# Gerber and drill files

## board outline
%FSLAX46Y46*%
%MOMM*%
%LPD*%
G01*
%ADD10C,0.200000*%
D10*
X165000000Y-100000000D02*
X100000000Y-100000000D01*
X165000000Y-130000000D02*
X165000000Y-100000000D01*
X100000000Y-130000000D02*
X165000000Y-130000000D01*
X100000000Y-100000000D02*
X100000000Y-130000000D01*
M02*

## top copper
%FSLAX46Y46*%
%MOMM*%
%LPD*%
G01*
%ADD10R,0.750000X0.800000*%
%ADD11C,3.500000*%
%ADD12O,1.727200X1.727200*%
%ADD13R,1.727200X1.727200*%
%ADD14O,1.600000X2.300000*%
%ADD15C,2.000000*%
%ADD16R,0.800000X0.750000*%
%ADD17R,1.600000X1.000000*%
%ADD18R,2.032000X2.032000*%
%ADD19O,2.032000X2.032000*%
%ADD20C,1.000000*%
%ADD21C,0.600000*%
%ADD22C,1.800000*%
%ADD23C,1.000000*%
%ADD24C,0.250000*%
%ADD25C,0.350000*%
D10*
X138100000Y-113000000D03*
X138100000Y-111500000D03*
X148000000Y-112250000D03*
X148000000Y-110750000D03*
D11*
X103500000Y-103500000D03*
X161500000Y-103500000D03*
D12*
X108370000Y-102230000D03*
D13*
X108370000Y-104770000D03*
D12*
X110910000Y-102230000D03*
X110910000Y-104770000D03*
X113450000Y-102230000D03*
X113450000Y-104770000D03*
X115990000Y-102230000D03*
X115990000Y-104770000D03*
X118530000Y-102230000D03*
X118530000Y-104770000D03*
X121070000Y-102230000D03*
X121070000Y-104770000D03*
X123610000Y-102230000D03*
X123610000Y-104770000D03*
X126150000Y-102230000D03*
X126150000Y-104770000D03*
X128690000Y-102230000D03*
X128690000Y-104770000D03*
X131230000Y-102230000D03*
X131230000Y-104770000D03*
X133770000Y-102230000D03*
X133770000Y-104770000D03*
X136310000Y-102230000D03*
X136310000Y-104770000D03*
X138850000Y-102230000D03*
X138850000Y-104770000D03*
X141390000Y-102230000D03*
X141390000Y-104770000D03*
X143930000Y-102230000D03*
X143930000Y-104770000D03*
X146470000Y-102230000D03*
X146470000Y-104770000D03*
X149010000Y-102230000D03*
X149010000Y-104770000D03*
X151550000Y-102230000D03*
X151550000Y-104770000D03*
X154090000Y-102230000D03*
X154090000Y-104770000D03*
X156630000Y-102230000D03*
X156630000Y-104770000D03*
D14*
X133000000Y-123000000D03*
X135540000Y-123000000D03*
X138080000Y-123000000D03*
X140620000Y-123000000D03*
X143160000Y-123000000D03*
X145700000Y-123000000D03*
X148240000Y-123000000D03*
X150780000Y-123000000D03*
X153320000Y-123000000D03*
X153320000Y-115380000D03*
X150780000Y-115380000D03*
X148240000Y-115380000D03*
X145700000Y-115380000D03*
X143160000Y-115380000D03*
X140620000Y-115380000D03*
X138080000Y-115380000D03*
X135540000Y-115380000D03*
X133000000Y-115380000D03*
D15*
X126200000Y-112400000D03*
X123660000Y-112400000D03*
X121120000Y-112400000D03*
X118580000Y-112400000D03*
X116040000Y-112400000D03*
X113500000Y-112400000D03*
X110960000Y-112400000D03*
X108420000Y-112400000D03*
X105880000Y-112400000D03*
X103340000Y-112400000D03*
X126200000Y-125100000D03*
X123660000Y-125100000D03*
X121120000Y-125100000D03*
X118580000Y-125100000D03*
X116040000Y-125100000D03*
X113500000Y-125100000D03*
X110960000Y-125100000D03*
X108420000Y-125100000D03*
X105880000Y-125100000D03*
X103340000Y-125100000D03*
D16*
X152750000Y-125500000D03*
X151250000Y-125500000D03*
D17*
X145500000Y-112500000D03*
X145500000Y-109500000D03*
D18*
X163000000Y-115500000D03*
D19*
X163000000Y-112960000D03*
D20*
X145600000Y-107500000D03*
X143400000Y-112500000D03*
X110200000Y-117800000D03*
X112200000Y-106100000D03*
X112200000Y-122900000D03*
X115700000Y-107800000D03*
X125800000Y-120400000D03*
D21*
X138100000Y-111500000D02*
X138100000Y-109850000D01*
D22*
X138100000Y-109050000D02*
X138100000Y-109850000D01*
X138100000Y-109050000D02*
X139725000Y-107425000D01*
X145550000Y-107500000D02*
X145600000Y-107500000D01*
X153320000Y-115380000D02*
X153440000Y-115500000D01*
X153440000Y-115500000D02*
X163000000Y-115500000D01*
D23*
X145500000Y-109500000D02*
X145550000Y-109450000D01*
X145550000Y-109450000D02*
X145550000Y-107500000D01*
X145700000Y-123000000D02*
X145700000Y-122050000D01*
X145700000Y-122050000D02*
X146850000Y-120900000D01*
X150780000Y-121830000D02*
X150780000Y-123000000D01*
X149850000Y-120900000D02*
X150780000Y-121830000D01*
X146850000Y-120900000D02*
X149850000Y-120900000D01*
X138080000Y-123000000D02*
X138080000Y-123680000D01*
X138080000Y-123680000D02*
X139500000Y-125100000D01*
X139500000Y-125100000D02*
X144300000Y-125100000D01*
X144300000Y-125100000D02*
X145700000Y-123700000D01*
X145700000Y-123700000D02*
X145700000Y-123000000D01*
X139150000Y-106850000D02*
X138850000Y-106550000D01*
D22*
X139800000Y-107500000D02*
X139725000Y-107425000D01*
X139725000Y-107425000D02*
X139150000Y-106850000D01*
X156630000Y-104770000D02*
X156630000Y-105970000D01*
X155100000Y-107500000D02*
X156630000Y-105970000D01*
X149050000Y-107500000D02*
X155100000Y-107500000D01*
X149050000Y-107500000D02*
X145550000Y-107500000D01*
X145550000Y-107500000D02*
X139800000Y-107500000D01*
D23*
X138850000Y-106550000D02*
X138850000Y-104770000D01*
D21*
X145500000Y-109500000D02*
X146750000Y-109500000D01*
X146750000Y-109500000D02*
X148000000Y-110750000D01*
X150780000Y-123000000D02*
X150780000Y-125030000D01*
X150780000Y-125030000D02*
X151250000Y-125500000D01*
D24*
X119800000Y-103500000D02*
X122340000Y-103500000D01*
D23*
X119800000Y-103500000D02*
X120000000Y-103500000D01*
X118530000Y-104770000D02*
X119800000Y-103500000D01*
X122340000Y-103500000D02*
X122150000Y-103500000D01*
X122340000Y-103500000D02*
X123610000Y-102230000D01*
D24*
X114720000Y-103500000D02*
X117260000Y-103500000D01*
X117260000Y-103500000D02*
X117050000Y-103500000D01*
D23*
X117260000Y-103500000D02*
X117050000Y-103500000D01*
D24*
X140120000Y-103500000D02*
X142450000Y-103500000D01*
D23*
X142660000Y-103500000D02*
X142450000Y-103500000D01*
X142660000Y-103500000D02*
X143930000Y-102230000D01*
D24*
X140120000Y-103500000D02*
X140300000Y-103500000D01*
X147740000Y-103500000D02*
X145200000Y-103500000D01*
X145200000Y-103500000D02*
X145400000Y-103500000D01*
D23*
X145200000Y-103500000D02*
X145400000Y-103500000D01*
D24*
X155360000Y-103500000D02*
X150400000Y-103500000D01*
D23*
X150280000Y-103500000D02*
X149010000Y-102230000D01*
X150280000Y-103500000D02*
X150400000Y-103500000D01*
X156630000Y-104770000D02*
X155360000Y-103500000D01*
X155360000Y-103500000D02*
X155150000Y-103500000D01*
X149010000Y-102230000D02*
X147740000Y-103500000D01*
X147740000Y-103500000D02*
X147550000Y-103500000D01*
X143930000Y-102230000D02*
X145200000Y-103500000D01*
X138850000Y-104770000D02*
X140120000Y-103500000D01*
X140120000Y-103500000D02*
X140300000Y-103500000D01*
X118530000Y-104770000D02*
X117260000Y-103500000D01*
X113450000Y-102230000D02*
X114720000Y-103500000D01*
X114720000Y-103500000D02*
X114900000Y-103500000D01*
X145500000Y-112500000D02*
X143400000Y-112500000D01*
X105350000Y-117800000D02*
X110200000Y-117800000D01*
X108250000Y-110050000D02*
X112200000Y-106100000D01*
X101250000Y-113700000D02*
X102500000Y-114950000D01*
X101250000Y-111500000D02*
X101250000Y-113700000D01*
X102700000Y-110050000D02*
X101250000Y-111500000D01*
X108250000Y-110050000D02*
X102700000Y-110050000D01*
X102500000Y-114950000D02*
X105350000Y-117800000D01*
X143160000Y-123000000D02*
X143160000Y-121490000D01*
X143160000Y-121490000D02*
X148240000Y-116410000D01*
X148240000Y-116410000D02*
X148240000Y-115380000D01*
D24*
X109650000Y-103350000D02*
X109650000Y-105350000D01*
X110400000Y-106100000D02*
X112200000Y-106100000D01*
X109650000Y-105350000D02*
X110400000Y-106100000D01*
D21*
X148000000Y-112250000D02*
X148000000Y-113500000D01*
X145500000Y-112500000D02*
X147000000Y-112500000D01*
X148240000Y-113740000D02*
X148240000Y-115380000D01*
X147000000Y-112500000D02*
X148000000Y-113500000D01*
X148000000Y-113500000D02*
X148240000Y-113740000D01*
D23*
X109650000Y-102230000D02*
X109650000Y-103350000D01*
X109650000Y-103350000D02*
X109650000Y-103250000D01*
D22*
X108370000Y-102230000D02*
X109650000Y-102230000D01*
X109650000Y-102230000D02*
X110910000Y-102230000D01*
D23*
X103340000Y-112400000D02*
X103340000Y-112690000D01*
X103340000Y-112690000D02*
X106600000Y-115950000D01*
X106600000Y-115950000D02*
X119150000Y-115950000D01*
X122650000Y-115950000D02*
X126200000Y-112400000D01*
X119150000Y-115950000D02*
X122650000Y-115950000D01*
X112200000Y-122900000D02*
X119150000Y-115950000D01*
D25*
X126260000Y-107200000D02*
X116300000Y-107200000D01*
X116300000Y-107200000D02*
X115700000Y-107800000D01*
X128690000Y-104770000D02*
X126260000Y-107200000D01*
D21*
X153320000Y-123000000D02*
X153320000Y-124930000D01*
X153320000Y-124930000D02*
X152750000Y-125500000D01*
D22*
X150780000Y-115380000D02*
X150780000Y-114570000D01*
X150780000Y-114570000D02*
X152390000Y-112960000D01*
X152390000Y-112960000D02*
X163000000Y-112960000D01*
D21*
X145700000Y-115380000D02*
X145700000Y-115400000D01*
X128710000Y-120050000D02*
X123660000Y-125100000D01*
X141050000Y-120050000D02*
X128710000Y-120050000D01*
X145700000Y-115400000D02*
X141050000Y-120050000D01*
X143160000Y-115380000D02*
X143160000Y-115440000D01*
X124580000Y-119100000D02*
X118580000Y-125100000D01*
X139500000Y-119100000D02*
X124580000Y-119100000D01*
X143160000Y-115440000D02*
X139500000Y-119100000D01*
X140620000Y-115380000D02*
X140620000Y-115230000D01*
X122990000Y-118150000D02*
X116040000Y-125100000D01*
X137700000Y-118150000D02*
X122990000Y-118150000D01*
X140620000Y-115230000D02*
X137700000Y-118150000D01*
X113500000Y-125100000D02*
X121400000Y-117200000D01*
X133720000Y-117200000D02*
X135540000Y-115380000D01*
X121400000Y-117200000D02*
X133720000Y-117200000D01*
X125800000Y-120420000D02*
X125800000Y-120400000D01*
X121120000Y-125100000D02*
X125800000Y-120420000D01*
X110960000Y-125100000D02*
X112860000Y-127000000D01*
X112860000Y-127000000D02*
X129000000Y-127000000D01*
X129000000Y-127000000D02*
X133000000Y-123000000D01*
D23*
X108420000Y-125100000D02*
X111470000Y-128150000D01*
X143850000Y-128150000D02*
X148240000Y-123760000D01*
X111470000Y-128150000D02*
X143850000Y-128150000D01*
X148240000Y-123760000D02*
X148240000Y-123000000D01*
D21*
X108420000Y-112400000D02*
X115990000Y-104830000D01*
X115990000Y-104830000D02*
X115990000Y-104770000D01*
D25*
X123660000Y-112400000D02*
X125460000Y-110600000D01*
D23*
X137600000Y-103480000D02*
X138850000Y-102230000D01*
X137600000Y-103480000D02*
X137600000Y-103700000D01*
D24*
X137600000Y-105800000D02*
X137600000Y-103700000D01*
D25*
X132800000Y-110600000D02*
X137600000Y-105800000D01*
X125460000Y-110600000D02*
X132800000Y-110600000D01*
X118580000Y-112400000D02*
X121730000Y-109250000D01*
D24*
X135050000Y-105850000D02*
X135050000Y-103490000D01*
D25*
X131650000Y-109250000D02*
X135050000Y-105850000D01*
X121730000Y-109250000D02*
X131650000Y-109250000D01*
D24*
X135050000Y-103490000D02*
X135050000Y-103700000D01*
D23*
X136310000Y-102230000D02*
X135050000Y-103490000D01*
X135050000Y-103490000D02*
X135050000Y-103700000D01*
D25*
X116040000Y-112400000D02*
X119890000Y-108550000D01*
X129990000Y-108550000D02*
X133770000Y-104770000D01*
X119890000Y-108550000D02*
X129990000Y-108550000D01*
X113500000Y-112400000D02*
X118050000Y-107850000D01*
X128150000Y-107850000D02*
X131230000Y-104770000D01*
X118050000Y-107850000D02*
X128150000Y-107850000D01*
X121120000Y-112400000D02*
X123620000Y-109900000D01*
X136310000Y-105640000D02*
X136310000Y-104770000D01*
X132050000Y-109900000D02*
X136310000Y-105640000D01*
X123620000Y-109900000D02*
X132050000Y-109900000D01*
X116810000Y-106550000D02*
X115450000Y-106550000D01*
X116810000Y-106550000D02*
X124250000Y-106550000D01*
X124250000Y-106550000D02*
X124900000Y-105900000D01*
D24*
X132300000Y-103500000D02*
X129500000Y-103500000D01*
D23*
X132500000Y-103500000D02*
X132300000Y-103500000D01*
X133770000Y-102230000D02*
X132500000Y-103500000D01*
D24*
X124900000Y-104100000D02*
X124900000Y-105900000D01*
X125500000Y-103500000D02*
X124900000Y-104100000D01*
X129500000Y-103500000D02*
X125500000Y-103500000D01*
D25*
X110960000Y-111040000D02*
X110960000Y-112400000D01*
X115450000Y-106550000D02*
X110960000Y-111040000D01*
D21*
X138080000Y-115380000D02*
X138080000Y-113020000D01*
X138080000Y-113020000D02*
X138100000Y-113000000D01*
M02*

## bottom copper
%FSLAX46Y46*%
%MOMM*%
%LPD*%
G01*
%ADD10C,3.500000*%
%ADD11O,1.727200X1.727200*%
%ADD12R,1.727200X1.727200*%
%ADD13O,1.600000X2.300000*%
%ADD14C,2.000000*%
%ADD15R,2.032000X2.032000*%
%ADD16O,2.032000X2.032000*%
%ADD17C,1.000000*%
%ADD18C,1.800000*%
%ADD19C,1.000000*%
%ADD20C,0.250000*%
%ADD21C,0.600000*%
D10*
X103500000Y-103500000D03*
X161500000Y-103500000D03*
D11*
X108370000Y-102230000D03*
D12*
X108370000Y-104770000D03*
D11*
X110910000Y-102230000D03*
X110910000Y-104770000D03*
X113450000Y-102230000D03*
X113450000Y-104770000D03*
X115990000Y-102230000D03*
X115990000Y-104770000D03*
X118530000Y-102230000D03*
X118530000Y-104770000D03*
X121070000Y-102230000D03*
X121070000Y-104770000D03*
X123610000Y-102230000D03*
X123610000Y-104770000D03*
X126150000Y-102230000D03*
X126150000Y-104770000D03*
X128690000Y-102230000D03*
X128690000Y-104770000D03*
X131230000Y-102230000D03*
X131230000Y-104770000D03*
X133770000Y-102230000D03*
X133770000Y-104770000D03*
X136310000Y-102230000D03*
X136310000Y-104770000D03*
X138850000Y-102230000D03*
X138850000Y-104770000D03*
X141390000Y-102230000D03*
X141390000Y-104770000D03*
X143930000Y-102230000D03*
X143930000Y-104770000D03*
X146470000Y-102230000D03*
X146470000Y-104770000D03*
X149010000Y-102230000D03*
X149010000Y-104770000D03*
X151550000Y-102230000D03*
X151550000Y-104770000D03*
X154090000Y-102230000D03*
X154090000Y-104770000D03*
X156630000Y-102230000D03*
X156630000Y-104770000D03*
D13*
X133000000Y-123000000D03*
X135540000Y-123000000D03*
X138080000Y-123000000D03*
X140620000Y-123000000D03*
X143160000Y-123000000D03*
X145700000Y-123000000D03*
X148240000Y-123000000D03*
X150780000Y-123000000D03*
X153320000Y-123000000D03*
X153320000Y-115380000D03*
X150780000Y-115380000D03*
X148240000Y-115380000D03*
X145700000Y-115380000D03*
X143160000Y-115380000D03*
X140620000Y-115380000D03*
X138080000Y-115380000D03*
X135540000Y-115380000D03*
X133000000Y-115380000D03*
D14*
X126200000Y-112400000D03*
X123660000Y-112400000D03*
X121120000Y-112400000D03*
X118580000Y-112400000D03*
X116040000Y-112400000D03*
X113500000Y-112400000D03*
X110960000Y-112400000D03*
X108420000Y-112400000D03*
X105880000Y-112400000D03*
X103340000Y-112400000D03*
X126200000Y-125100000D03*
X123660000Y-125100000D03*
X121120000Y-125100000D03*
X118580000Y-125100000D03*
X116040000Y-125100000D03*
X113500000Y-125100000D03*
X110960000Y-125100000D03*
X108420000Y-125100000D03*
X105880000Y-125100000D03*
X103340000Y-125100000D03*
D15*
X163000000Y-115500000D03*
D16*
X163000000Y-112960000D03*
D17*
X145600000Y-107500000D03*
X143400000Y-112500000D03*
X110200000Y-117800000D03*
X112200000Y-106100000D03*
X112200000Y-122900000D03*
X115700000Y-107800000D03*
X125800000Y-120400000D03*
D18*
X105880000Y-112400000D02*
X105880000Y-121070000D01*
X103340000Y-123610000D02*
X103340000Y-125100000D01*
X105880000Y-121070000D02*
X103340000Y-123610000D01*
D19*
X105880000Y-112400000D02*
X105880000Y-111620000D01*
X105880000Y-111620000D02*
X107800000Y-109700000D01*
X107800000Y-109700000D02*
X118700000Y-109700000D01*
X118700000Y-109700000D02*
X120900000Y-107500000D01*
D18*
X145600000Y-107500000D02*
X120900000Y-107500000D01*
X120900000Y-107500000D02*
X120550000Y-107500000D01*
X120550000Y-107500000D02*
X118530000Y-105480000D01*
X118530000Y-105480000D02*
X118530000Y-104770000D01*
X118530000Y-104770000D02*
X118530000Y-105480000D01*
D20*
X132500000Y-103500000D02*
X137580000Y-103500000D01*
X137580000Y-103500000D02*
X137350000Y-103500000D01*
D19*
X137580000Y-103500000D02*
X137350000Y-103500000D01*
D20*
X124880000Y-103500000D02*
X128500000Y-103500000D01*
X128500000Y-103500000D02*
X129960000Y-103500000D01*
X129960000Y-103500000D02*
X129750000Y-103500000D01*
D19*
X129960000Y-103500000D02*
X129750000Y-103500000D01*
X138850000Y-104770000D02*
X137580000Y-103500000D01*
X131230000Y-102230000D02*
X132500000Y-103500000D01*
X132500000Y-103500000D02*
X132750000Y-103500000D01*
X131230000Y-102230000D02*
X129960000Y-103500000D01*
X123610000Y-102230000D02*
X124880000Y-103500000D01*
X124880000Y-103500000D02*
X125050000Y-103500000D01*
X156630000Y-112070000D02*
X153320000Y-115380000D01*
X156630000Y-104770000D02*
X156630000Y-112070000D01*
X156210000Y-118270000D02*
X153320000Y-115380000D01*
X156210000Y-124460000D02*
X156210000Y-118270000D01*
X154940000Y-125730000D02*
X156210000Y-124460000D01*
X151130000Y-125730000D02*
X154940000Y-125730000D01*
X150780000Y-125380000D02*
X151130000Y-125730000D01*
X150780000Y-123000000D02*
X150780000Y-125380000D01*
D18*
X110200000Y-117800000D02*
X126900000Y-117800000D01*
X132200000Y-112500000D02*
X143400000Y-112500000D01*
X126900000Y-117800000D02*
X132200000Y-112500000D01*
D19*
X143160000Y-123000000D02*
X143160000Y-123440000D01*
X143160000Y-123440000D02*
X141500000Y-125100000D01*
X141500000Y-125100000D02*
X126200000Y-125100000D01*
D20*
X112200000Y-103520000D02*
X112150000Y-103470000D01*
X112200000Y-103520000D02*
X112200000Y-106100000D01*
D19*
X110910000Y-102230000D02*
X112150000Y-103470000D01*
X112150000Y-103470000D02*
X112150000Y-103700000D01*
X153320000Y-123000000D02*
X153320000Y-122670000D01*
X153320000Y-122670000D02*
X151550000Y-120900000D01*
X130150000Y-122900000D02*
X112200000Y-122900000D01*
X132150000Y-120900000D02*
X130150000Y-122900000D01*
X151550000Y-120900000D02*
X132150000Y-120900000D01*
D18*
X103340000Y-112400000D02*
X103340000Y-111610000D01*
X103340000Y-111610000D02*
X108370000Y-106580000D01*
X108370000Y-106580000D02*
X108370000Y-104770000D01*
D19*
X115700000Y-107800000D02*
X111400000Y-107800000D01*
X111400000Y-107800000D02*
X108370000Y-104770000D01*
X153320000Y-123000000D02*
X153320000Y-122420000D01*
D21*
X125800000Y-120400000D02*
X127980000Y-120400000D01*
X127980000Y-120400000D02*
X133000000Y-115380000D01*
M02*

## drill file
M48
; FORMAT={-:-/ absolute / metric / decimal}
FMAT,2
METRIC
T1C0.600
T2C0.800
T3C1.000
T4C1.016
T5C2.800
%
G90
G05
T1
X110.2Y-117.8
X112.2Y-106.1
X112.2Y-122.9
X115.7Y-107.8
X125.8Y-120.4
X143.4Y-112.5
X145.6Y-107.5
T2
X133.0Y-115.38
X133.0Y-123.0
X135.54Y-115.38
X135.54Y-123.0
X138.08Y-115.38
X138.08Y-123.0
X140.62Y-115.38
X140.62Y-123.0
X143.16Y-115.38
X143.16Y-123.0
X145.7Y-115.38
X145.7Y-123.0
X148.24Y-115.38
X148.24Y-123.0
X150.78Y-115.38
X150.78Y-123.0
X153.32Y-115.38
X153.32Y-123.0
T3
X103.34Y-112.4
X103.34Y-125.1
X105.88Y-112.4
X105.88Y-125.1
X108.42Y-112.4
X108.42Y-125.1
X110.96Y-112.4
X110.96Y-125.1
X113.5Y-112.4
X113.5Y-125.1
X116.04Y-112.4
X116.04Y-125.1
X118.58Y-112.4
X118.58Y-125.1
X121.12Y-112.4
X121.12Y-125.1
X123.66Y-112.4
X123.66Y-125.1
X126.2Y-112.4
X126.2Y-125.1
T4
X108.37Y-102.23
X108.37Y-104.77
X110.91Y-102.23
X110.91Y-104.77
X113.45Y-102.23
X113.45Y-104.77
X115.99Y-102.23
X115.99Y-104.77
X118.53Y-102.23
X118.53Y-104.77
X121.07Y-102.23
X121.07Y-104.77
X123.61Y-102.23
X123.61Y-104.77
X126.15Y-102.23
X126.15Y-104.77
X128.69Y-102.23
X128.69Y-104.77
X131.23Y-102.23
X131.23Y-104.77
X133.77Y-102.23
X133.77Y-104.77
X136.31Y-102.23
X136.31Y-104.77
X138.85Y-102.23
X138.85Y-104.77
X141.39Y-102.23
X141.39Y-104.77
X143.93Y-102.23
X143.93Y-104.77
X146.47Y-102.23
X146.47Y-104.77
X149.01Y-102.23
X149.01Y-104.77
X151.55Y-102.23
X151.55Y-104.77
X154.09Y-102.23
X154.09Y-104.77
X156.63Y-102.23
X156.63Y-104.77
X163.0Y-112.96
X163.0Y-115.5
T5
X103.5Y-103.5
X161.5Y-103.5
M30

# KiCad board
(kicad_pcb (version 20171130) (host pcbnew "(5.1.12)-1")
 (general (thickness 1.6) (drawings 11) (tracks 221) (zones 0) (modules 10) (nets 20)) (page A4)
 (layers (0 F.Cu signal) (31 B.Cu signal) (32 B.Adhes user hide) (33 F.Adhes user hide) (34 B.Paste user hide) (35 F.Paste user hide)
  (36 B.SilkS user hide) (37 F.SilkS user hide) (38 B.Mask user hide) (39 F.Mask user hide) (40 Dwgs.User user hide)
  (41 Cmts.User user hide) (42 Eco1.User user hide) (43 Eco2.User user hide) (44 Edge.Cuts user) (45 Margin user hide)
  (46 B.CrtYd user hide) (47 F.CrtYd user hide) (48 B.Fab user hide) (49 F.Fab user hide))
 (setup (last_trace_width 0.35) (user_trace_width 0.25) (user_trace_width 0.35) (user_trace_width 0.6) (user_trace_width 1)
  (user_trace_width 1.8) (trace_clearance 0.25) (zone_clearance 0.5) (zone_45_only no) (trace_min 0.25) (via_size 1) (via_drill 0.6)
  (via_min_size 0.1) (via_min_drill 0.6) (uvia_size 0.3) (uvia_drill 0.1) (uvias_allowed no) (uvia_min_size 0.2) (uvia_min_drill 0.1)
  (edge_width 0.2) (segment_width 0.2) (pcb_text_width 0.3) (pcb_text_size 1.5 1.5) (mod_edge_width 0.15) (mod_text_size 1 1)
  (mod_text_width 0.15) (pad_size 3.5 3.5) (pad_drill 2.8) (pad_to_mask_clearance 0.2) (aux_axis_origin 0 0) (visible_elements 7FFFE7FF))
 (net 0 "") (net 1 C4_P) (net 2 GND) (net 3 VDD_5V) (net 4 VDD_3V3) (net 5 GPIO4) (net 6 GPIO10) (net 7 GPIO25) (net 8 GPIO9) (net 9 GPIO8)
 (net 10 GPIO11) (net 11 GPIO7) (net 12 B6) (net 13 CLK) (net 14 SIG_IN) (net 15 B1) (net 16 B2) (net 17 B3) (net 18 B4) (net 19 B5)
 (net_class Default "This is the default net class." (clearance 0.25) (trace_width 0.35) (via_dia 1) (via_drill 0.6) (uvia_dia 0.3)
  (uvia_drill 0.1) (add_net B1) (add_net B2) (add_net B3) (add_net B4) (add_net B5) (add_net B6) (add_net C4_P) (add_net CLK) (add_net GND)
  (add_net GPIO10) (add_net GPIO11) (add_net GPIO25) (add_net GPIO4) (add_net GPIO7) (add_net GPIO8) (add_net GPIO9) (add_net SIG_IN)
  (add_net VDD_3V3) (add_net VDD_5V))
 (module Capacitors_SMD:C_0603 (layer F.Cu) (at 138.1 112.25 90)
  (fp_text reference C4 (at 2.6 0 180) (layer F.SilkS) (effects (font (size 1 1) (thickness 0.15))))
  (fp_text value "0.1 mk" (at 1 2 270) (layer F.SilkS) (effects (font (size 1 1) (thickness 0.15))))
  (pad 1 smd rect (at -0.75 0 90) (size 0.8 0.75) (layers F.Cu F.Paste F.Mask) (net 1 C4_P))
  (pad 2 smd rect (at 0.75 0 90) (size 0.8 0.75) (layers F.Cu F.Paste F.Mask) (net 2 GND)))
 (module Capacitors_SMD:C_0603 (layer F.Cu) (at 148 111.5 90)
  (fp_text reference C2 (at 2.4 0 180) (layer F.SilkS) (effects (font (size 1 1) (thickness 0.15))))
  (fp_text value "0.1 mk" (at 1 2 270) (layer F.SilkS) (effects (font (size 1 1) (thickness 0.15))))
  (pad 1 smd rect (at -0.75 0 90) (size 0.8 0.75) (layers F.Cu F.Paste F.Mask) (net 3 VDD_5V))
  (pad 2 smd rect (at 0.75 0 90) (size 0.8 0.75) (layers F.Cu F.Paste F.Mask) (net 2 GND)))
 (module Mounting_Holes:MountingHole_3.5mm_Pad (layer F.Cu) (at 103.5 103.5)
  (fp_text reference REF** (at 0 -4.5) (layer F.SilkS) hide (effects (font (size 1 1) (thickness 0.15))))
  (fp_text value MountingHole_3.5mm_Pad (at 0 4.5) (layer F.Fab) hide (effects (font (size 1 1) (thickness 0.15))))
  (pad "" np_thru_hole circle (at 0 0) (size 3.5 3.5) (drill 2.8) (layers *.Cu *.Mask)))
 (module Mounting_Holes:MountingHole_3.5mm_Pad (layer F.Cu) (at 161.5 103.5)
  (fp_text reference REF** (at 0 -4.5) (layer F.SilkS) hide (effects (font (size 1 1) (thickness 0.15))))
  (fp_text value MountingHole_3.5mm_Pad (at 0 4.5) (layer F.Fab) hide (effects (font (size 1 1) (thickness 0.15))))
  (pad "" np_thru_hole circle (at 0 0) (size 3.5 3.5) (drill 2.8) (layers *.Cu *.Mask)))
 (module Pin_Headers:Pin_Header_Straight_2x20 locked (layer B.Cu) (at 108.37 102.23 270)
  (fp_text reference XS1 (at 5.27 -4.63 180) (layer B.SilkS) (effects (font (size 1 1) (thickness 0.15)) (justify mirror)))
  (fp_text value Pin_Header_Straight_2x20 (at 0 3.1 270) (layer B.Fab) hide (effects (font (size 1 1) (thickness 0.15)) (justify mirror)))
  (pad 2 thru_hole oval (at 0 0 270) (size 1.7272 1.7272) (drill 1.016) (layers *.Cu *.Mask B.SilkS) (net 3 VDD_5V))
  (pad 1 thru_hole rect (at 2.54 0 270) (size 1.7272 1.7272) (drill 1.016) (layers *.Cu *.Mask B.SilkS) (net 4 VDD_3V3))
  (pad 4 thru_hole oval (at 0 -2.54 270) (size 1.7272 1.7272) (drill 1.016) (layers *.Cu *.Mask B.SilkS) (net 3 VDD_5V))
  (pad 3 thru_hole oval (at 2.54 -2.54 270) (size 1.7272 1.7272) (drill 1.016) (layers *.Cu *.Mask B.SilkS))
  (pad 6 thru_hole oval (at 0 -5.08 270) (size 1.7272 1.7272) (drill 1.016) (layers *.Cu *.Mask B.SilkS) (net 2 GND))
  (pad 5 thru_hole oval (at 2.54 -5.08 270) (size 1.7272 1.7272) (drill 1.016) (layers *.Cu *.Mask B.SilkS))
  (pad 8 thru_hole oval (at 0 -7.62 270) (size 1.7272 1.7272) (drill 1.016) (layers *.Cu *.Mask B.SilkS))
  (pad 7 thru_hole oval (at 2.54 -7.62 270) (size 1.7272 1.7272) (drill 1.016) (layers *.Cu *.Mask B.SilkS) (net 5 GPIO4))
  (pad 10 thru_hole oval (at 0 -10.16 270) (size 1.7272 1.7272) (drill 1.016) (layers *.Cu *.Mask B.SilkS))
  (pad 9 thru_hole oval (at 2.54 -10.16 270) (size 1.7272 1.7272) (drill 1.016) (layers *.Cu *.Mask B.SilkS) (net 2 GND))
  (pad 12 thru_hole oval (at 0 -12.7 270) (size 1.7272 1.7272) (drill 1.016) (layers *.Cu *.Mask B.SilkS))
  (pad 11 thru_hole oval (at 2.54 -12.7 270) (size 1.7272 1.7272) (drill 1.016) (layers *.Cu *.Mask B.SilkS))
  (pad 14 thru_hole oval (at 0 -15.24 270) (size 1.7272 1.7272) (drill 1.016) (layers *.Cu *.Mask B.SilkS) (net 2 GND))
  (pad 13 thru_hole oval (at 2.54 -15.24 270) (size 1.7272 1.7272) (drill 1.016) (layers *.Cu *.Mask B.SilkS))
  (pad 16 thru_hole oval (at 0 -17.78 270) (size 1.7272 1.7272) (drill 1.016) (layers *.Cu *.Mask B.SilkS))
  (pad 15 thru_hole oval (at 2.54 -17.78 270) (size 1.7272 1.7272) (drill 1.016) (layers *.Cu *.Mask B.SilkS))
  (pad 18 thru_hole oval (at 0 -20.32 270) (size 1.7272 1.7272) (drill 1.016) (layers *.Cu *.Mask B.SilkS))
  (pad 17 thru_hole oval (at 2.54 -20.32 270) (size 1.7272 1.7272) (drill 1.016) (layers *.Cu *.Mask B.SilkS) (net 4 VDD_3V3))
  (pad 20 thru_hole oval (at 0 -22.86 270) (size 1.7272 1.7272) (drill 1.016) (layers *.Cu *.Mask B.SilkS) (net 2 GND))
  (pad 19 thru_hole oval (at 2.54 -22.86 270) (size 1.7272 1.7272) (drill 1.016) (layers *.Cu *.Mask B.SilkS) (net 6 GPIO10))
  (pad 22 thru_hole oval (at 0 -25.4 270) (size 1.7272 1.7272) (drill 1.016) (layers *.Cu *.Mask B.SilkS) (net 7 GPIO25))
  (pad 21 thru_hole oval (at 2.54 -25.4 270) (size 1.7272 1.7272) (drill 1.016) (layers *.Cu *.Mask B.SilkS) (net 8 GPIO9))
  (pad 24 thru_hole oval (at 0 -27.94 270) (size 1.7272 1.7272) (drill 1.016) (layers *.Cu *.Mask B.SilkS) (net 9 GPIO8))
  (pad 23 thru_hole oval (at 2.54 -27.94 270) (size 1.7272 1.7272) (drill 1.016) (layers *.Cu *.Mask B.SilkS) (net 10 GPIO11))
  (pad 26 thru_hole oval (at 0 -30.48 270) (size 1.7272 1.7272) (drill 1.016) (layers *.Cu *.Mask B.SilkS) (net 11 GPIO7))
  (pad 25 thru_hole oval (at 2.54 -30.48 270) (size 1.7272 1.7272) (drill 1.016) (layers *.Cu *.Mask B.SilkS) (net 2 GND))
  (pad 28 thru_hole oval (at 0 -33.02 270) (size 1.7272 1.7272) (drill 1.016) (layers *.Cu *.Mask B.SilkS))
  (pad 27 thru_hole oval (at 2.54 -33.02 270) (size 1.7272 1.7272) (drill 1.016) (layers *.Cu *.Mask B.SilkS))
  (pad 30 thru_hole oval (at 0 -35.56 270) (size 1.7272 1.7272) (drill 1.016) (layers *.Cu *.Mask B.SilkS) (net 2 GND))
  (pad 29 thru_hole oval (at 2.54 -35.56 270) (size 1.7272 1.7272) (drill 1.016) (layers *.Cu *.Mask B.SilkS))
  (pad 32 thru_hole oval (at 0 -38.1 270) (size 1.7272 1.7272) (drill 1.016) (layers *.Cu *.Mask B.SilkS))
  (pad 31 thru_hole oval (at 2.54 -38.1 270) (size 1.7272 1.7272) (drill 1.016) (layers *.Cu *.Mask B.SilkS))
  (pad 34 thru_hole oval (at 0 -40.64 270) (size 1.7272 1.7272) (drill 1.016) (layers *.Cu *.Mask B.SilkS) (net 2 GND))
  (pad 33 thru_hole oval (at 2.54 -40.64 270) (size 1.7272 1.7272) (drill 1.016) (layers *.Cu *.Mask B.SilkS))
  (pad 36 thru_hole oval (at 0 -43.18 270) (size 1.7272 1.7272) (drill 1.016) (layers *.Cu *.Mask B.SilkS))
  (pad 35 thru_hole oval (at 2.54 -43.18 270) (size 1.7272 1.7272) (drill 1.016) (layers *.Cu *.Mask B.SilkS))
  (pad 38 thru_hole oval (at 0 -45.72 270) (size 1.7272 1.7272) (drill 1.016) (layers *.Cu *.Mask B.SilkS))
  (pad 37 thru_hole oval (at 2.54 -45.72 270) (size 1.7272 1.7272) (drill 1.016) (layers *.Cu *.Mask B.SilkS))
  (pad 40 thru_hole oval (at 0 -48.26 270) (size 1.7272 1.7272) (drill 1.016) (layers *.Cu *.Mask B.SilkS))
  (pad 39 thru_hole oval (at 2.54 -48.26 270) (size 1.7272 1.7272) (drill 1.016) (layers *.Cu *.Mask B.SilkS) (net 2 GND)))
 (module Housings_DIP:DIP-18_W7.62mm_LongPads (layer F.Cu) (at 133 123 90)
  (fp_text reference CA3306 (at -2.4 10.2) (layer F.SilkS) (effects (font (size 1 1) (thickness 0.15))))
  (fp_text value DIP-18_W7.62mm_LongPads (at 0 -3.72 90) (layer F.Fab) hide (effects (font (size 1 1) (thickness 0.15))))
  (pad 1 thru_hole oval (at 0 0 90) (size 2.3 1.6) (drill 0.8) (layers *.Cu *.Mask F.SilkS) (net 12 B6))
  (pad 2 thru_hole oval (at 0 2.54 90) (size 2.3 1.6) (drill 0.8) (layers *.Cu *.Mask F.SilkS))
  (pad 3 thru_hole oval (at 0 5.08 90) (size 2.3 1.6) (drill 0.8) (layers *.Cu *.Mask F.SilkS) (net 2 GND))
  (pad 4 thru_hole oval (at 0 7.62 90) (size 2.3 1.6) (drill 0.8) (layers *.Cu *.Mask F.SilkS))
  (pad 5 thru_hole oval (at 0 10.16 90) (size 2.3 1.6) (drill 0.8) (layers *.Cu *.Mask F.SilkS) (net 3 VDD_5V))
  (pad 6 thru_hole oval (at 0 12.7 90) (size 2.3 1.6) (drill 0.8) (layers *.Cu *.Mask F.SilkS) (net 2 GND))
  (pad 7 thru_hole oval (at 0 15.24 90) (size 2.3 1.6) (drill 0.8) (layers *.Cu *.Mask F.SilkS) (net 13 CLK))
  (pad 8 thru_hole oval (at 0 17.78 90) (size 2.3 1.6) (drill 0.8) (layers *.Cu *.Mask F.SilkS) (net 2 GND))
  (pad 9 thru_hole oval (at 0 20.32 90) (size 2.3 1.6) (drill 0.8) (layers *.Cu *.Mask F.SilkS) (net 4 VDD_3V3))
  (pad 10 thru_hole oval (at 7.62 20.32 90) (size 2.3 1.6) (drill 0.8) (layers *.Cu *.Mask F.SilkS) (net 2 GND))
  (pad 11 thru_hole oval (at 7.62 17.78 90) (size 2.3 1.6) (drill 0.8) (layers *.Cu *.Mask F.SilkS) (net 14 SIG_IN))
  (pad 12 thru_hole oval (at 7.62 15.24 90) (size 2.3 1.6) (drill 0.8) (layers *.Cu *.Mask F.SilkS) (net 3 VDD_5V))
  (pad 13 thru_hole oval (at 7.62 12.7 90) (size 2.3 1.6) (drill 0.8) (layers *.Cu *.Mask F.SilkS) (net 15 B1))
  (pad 14 thru_hole oval (at 7.62 10.16 90) (size 2.3 1.6) (drill 0.8) (layers *.Cu *.Mask F.SilkS) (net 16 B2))
  (pad 15 thru_hole oval (at 7.62 7.62 90) (size 2.3 1.6) (drill 0.8) (layers *.Cu *.Mask F.SilkS) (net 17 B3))
  (pad 16 thru_hole oval (at 7.62 5.08 90) (size 2.3 1.6) (drill 0.8) (layers *.Cu *.Mask F.SilkS) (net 1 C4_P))
  (pad 17 thru_hole oval (at 7.62 2.54 90) (size 2.3 1.6) (drill 0.8) (layers *.Cu *.Mask F.SilkS) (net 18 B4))
  (pad 18 thru_hole oval (at 7.62 0 90) (size 2.3 1.6) (drill 0.8) (layers *.Cu *.Mask F.SilkS) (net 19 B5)))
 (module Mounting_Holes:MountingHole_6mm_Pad (layer F.Cu) (at 129 111 270)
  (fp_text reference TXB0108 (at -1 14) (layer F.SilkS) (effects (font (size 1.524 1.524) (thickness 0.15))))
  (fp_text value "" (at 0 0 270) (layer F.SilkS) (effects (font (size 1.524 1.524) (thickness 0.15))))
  (pad 1 thru_hole circle (at 1.4 2.8 270) (size 2 2) (drill 1) (layers *.Cu *.Mask F.SilkS) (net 4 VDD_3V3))
  (pad 2 thru_hole circle (at 1.4 5.34 270) (size 2 2) (drill 1) (layers *.Cu *.Mask F.SilkS) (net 11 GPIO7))
  (pad 3 thru_hole circle (at 1.4 7.88 270) (size 2 2) (drill 1) (layers *.Cu *.Mask F.SilkS) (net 10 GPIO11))
  (pad 4 thru_hole circle (at 1.4 10.42 270) (size 2 2) (drill 1) (layers *.Cu *.Mask F.SilkS) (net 9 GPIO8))
  (pad 5 thru_hole circle (at 1.4 12.96 270) (size 2 2) (drill 1) (layers *.Cu *.Mask F.SilkS) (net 8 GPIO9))
  (pad 6 thru_hole circle (at 1.4 15.5 270) (size 2 2) (drill 1) (layers *.Cu *.Mask F.SilkS) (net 6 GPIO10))
  (pad 7 thru_hole circle (at 1.4 18.04 270) (size 2 2) (drill 1) (layers *.Cu *.Mask F.SilkS) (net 7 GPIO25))
  (pad 8 thru_hole circle (at 1.4 20.58 270) (size 2 2) (drill 1) (layers *.Cu *.Mask F.SilkS) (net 5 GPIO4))
  (pad 9 thru_hole circle (at 1.4 23.12 270) (size 2 2) (drill 1) (layers *.Cu *.Mask F.SilkS) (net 2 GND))
  (pad 10 thru_hole circle (at 1.4 25.66 270) (size 2 2) (drill 1) (layers *.Cu *.Mask F.SilkS) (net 4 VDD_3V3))
  (pad 20 thru_hole circle (at 14.1 2.8 270) (size 2 2) (drill 1) (layers *.Cu *.Mask F.SilkS) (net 3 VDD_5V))
  (pad 19 thru_hole circle (at 14.1 5.34 270) (size 2 2) (drill 1) (layers *.Cu *.Mask F.SilkS) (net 15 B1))
  (pad 18 thru_hole circle (at 14.1 7.88 270) (size 2 2) (drill 1) (layers *.Cu *.Mask F.SilkS) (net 19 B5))
  (pad 17 thru_hole circle (at 14.1 10.42 270) (size 2 2) (drill 1) (layers *.Cu *.Mask F.SilkS) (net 16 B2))
  (pad 16 thru_hole circle (at 14.1 12.96 270) (size 2 2) (drill 1) (layers *.Cu *.Mask F.SilkS) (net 17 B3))
  (pad 15 thru_hole circle (at 14.1 15.5 270) (size 2 2) (drill 1) (layers *.Cu *.Mask F.SilkS) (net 18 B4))
  (pad 14 thru_hole circle (at 14.1 18.04 270) (size 2 2) (drill 1) (layers *.Cu *.Mask F.SilkS) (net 12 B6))
  (pad 13 thru_hole circle (at 14.1 20.58 270) (size 2 2) (drill 1) (layers *.Cu *.Mask F.SilkS) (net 13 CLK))
  (pad 12 thru_hole circle (at 14.1 23.12 270) (size 2 2) (drill 1) (layers *.Cu *.Mask F.SilkS))
  (pad 11 thru_hole circle (at 14.1 25.66 270) (size 2 2) (drill 1) (layers *.Cu *.Mask F.SilkS) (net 2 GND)))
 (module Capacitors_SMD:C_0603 (layer F.Cu) (at 152 125.5 180)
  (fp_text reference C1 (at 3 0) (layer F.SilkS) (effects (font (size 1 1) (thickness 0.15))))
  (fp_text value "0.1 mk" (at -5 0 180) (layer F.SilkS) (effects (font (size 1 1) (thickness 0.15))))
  (pad 1 smd rect (at -0.75 0 180) (size 0.8 0.75) (layers F.Cu F.Paste F.Mask) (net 4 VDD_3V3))
  (pad 2 smd rect (at 0.75 0 180) (size 0.8 0.75) (layers F.Cu F.Paste F.Mask) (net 2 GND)))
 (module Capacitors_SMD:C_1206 (layer F.Cu) (at 145.5 111 90)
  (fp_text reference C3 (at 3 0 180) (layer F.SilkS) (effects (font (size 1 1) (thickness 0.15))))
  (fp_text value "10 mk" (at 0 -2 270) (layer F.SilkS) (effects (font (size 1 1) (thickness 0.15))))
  (pad 1 smd rect (at -1.5 0 90) (size 1 1.6) (layers F.Cu F.Paste F.Mask) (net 3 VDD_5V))
  (pad 2 smd rect (at 1.5 0 90) (size 1 1.6) (layers F.Cu F.Paste F.Mask) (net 2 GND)))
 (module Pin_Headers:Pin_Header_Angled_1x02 (layer B.Cu) (at 163 115.5)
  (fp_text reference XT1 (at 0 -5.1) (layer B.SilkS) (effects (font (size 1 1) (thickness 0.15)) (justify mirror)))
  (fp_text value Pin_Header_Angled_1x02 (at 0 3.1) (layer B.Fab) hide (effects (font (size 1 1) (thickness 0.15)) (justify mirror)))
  (pad 1 thru_hole rect (at 0 0) (size 2.032 2.032) (drill 1.016) (layers *.Cu *.Mask B.SilkS) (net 2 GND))
  (pad 2 thru_hole oval (at 0 -2.54) (size 2.032 2.032) (drill 1.016) (layers *.Cu *.Mask B.SilkS) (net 14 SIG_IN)))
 (gr_line (start 165 100) (end 100 100) (angle 90) (layer Edge.Cuts) (width 0.2))
 (gr_line (start 165 130) (end 165 100) (angle 90) (layer Edge.Cuts) (width 0.2))
 (gr_line (start 100 130) (end 165 130) (angle 90) (layer Edge.Cuts) (width 0.2))
 (gr_line (start 100 100) (end 100 130) (angle 90) (layer Edge.Cuts) (width 0.2))
 (segment (start 138.1 111.5) (end 138.1 109.85) (width 0.6) (layer F.Cu) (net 2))
 (segment (start 138.1 109.05) (end 138.1 109.85) (width 1.8) (layer F.Cu) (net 2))
 (segment (start 138.1 109.05) (end 139.725 107.425) (width 1.8) (layer F.Cu) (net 2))
 (segment (start 105.88 112.4) (end 105.88 121.07) (width 1.8) (layer B.Cu) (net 2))
 (segment (start 103.34 123.61) (end 103.34 125.1) (width 1.8) (layer B.Cu) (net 2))
 (segment (start 105.88 121.07) (end 103.34 123.61) (width 1.8) (layer B.Cu) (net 2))
 (segment (start 105.88 112.4) (end 105.88 111.62) (width 1) (layer B.Cu) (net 2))
 (segment (start 105.88 111.62) (end 107.8 109.7) (width 1) (layer B.Cu) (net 2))
 (segment (start 107.8 109.7) (end 118.7 109.7) (width 1) (layer B.Cu) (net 2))
 (segment (start 118.7 109.7) (end 120.9 107.5) (width 1) (layer B.Cu) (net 2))
 (segment (start 145.6 107.5) (end 120.9 107.5) (width 1.8) (layer B.Cu) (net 2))
 (segment (start 120.9 107.5) (end 120.55 107.5) (width 1.8) (layer B.Cu) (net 2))
 (via (at 145.6 107.5) (size 1) (drill 0.6) (layers F.Cu B.Cu) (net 2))
 (segment (start 145.55 107.5) (end 145.6 107.5) (width 1.8) (layer F.Cu) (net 2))
 (segment (start 120.55 107.5) (end 118.53 105.48) (width 1.8) (layer B.Cu) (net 2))
 (segment (start 118.53 105.48) (end 118.53 104.77) (width 1.8) (layer B.Cu) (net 2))
 (segment (start 118.53 104.77) (end 118.53 105.48) (width 1.8) (layer B.Cu) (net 2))
 (segment (start 153.32 115.38) (end 153.44 115.5) (width 1.8) (layer F.Cu) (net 2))
 (segment (start 153.44 115.5) (end 163 115.5) (width 1.8) (layer F.Cu) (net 2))
 (segment (start 145.5 109.5) (end 145.55 109.45) (width 1) (layer F.Cu) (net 2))
 (segment (start 145.55 109.45) (end 145.55 107.5) (width 1) (layer F.Cu) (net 2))
 (segment (start 145.7 123) (end 145.7 122.05) (width 1) (layer F.Cu) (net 2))
 (segment (start 145.7 122.05) (end 146.85 120.9) (width 1) (layer F.Cu) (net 2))
 (segment (start 150.78 121.83) (end 150.78 123) (width 1) (layer F.Cu) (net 2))
 (segment (start 149.85 120.9) (end 150.78 121.83) (width 1) (layer F.Cu) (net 2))
 (segment (start 146.85 120.9) (end 149.85 120.9) (width 1) (layer F.Cu) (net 2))
 (segment (start 138.08 123) (end 138.08 123.68) (width 1) (layer F.Cu) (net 2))
 (segment (start 138.08 123.68) (end 139.5 125.1) (width 1) (layer F.Cu) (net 2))
 (segment (start 139.5 125.1) (end 144.3 125.1) (width 1) (layer F.Cu) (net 2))
 (segment (start 144.3 125.1) (end 145.7 123.7) (width 1) (layer F.Cu) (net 2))
 (segment (start 145.7 123.7) (end 145.7 123) (width 1) (layer F.Cu) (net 2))
 (segment (start 139.15 106.85) (end 138.85 106.55) (width 1) (layer F.Cu) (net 2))
 (segment (start 139.8 107.5) (end 139.725 107.425) (width 1.8) (layer F.Cu) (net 2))
 (segment (start 139.725 107.425) (end 139.15 106.85) (width 1.8) (layer F.Cu) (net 2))
 (segment (start 156.63 104.77) (end 156.63 105.97) (width 1.8) (layer F.Cu) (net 2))
 (segment (start 155.1 107.5) (end 156.63 105.97) (width 1.8) (layer F.Cu) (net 2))
 (segment (start 149.05 107.5) (end 155.1 107.5) (width 1.8) (layer F.Cu) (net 2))
 (segment (start 149.05 107.5) (end 145.55 107.5) (width 1.8) (layer F.Cu) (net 2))
 (segment (start 145.55 107.5) (end 139.8 107.5) (width 1.8) (layer F.Cu) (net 2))
 (segment (start 138.85 106.55) (end 138.85 104.77) (width 1) (layer F.Cu) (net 2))
 (segment (start 145.5 109.5) (end 146.75 109.5) (width 0.6) (layer F.Cu) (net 2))
 (segment (start 146.75 109.5) (end 148 110.75) (width 0.6) (layer F.Cu) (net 2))
 (segment (start 150.78 123) (end 150.78 125.03) (width 0.6) (layer F.Cu) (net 2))
 (segment (start 150.78 125.03) (end 151.25 125.5) (width 0.6) (layer F.Cu) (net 2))
 (segment (start 132.5 103.5) (end 137.58 103.5) (width 0.25) (layer B.Cu) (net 2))
 (segment (start 137.58 103.5) (end 137.35 103.5) (width 0.25) (layer B.Cu) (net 2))
 (segment (start 137.58 103.5) (end 137.35 103.5) (width 1) (layer B.Cu) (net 2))
 (segment (start 124.88 103.5) (end 128.5 103.5) (width 0.25) (layer B.Cu) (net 2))
 (segment (start 128.5 103.5) (end 129.96 103.5) (width 0.25) (layer B.Cu) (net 2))
 (segment (start 129.96 103.5) (end 129.75 103.5) (width 0.25) (layer B.Cu) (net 2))
 (segment (start 129.96 103.5) (end 129.75 103.5) (width 1) (layer B.Cu) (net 2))
 (segment (start 119.8 103.5) (end 122.34 103.5) (width 0.25) (layer F.Cu) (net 2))
 (segment (start 119.8 103.5) (end 120 103.5) (width 1) (layer F.Cu) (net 2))
 (segment (start 118.53 104.77) (end 119.8 103.5) (width 1) (layer F.Cu) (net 2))
 (segment (start 122.34 103.5) (end 122.15 103.5) (width 1) (layer F.Cu) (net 2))
 (segment (start 122.34 103.5) (end 123.61 102.23) (width 1) (layer F.Cu) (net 2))
 (segment (start 114.72 103.5) (end 117.26 103.5) (width 0.25) (layer F.Cu) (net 2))
 (segment (start 117.26 103.5) (end 117.05 103.5) (width 0.25) (layer F.Cu) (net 2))
 (segment (start 117.26 103.5) (end 117.05 103.5) (width 1) (layer F.Cu) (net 2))
 (segment (start 140.12 103.5) (end 142.45 103.5) (width 0.25) (layer F.Cu) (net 2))
 (segment (start 142.66 103.5) (end 142.45 103.5) (width 1) (layer F.Cu) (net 2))
 (segment (start 142.66 103.5) (end 143.93 102.23) (width 1) (layer F.Cu) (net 2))
 (segment (start 140.12 103.5) (end 140.3 103.5) (width 0.25) (layer F.Cu) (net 2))
 (segment (start 147.74 103.5) (end 145.2 103.5) (width 0.25) (layer F.Cu) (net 2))
 (segment (start 145.2 103.5) (end 145.4 103.5) (width 0.25) (layer F.Cu) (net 2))
 (segment (start 145.2 103.5) (end 145.4 103.5) (width 1) (layer F.Cu) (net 2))
 (segment (start 155.36 103.5) (end 150.4 103.5) (width 0.25) (layer F.Cu) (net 2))
 (segment (start 150.28 103.5) (end 149.01 102.23) (width 1) (layer F.Cu) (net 2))
 (segment (start 150.28 103.5) (end 150.4 103.5) (width 1) (layer F.Cu) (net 2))
 (segment (start 156.63 104.77) (end 155.36 103.5) (width 1) (layer F.Cu) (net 2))
 (segment (start 155.36 103.5) (end 155.15 103.5) (width 1) (layer F.Cu) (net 2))
 (segment (start 149.01 102.23) (end 147.74 103.5) (width 1) (layer F.Cu) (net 2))
 (segment (start 147.74 103.5) (end 147.55 103.5) (width 1) (layer F.Cu) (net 2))
 (segment (start 143.93 102.23) (end 145.2 103.5) (width 1) (layer F.Cu) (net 2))
 (segment (start 138.85 104.77) (end 140.12 103.5) (width 1) (layer F.Cu) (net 2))
 (segment (start 140.12 103.5) (end 140.3 103.5) (width 1) (layer F.Cu) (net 2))
 (segment (start 138.85 104.77) (end 137.58 103.5) (width 1) (layer B.Cu) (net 2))
 (segment (start 131.23 102.23) (end 132.5 103.5) (width 1) (layer B.Cu) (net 2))
 (segment (start 132.5 103.5) (end 132.75 103.5) (width 1) (layer B.Cu) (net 2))
 (segment (start 131.23 102.23) (end 129.96 103.5) (width 1) (layer B.Cu) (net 2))
 (segment (start 123.61 102.23) (end 124.88 103.5) (width 1) (layer B.Cu) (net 2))
 (segment (start 124.88 103.5) (end 125.05 103.5) (width 1) (layer B.Cu) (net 2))
 (segment (start 118.53 104.77) (end 117.26 103.5) (width 1) (layer F.Cu) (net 2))
 (segment (start 113.45 102.23) (end 114.72 103.5) (width 1) (layer F.Cu) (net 2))
 (segment (start 114.72 103.5) (end 114.9 103.5) (width 1) (layer F.Cu) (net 2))
 (segment (start 156.63 112.07) (end 153.32 115.38) (width 1) (layer B.Cu) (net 2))
 (segment (start 156.63 104.77) (end 156.63 112.07) (width 1) (layer B.Cu) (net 2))
 (segment (start 156.21 118.27) (end 153.32 115.38) (width 1) (layer B.Cu) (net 2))
 (segment (start 156.21 124.46) (end 156.21 118.27) (width 1) (layer B.Cu) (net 2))
 (segment (start 154.94 125.73) (end 156.21 124.46) (width 1) (layer B.Cu) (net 2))
 (segment (start 151.13 125.73) (end 154.94 125.73) (width 1) (layer B.Cu) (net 2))
 (segment (start 150.78 125.38) (end 151.13 125.73) (width 1) (layer B.Cu) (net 2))
 (segment (start 150.78 123) (end 150.78 125.38) (width 1) (layer B.Cu) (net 2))
 (segment (start 110.2 117.8) (end 126.9 117.8) (width 1.8) (layer B.Cu) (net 3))
 (segment (start 145.5 112.5) (end 143.4 112.5) (width 1) (layer F.Cu) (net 3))
 (via (at 143.4 112.5) (size 1) (drill 0.6) (layers F.Cu B.Cu) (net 3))
 (segment (start 105.35 117.8) (end 110.2 117.8) (width 1) (layer F.Cu) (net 3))
 (via (at 110.2 117.8) (size 1) (drill 0.6) (layers F.Cu B.Cu) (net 3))
 (segment (start 108.25 110.05) (end 112.2 106.1) (width 1) (layer F.Cu) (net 3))
 (segment (start 101.25 113.7) (end 102.5 114.95) (width 1) (layer F.Cu) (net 3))
 (segment (start 101.25 111.5) (end 101.25 113.7) (width 1) (layer F.Cu) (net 3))
 (segment (start 102.7 110.05) (end 101.25 111.5) (width 1) (layer F.Cu) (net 3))
 (segment (start 108.25 110.05) (end 102.7 110.05) (width 1) (layer F.Cu) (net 3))
 (segment (start 102.5 114.95) (end 105.35 117.8) (width 1) (layer F.Cu) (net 3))
 (segment (start 132.2 112.5) (end 143.4 112.5) (width 1.8) (layer B.Cu) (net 3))
 (segment (start 126.9 117.8) (end 132.2 112.5) (width 1.8) (layer B.Cu) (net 3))
 (segment (start 143.16 123) (end 143.16 123.44) (width 1) (layer B.Cu) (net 3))
 (segment (start 143.16 123.44) (end 141.5 125.1) (width 1) (layer B.Cu) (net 3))
 (segment (start 141.5 125.1) (end 126.2 125.1) (width 1) (layer B.Cu) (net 3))
 (segment (start 143.16 123) (end 143.16 121.49) (width 1) (layer F.Cu) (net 3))
 (segment (start 143.16 121.49) (end 148.24 116.41) (width 1) (layer F.Cu) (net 3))
 (segment (start 148.24 116.41) (end 148.24 115.38) (width 1) (layer F.Cu) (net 3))
 (segment (start 109.65 103.35) (end 109.65 105.35) (width 0.25) (layer F.Cu) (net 3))
 (segment (start 110.4 106.1) (end 112.2 106.1) (width 0.25) (layer F.Cu) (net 3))
 (segment (start 109.65 105.35) (end 110.4 106.1) (width 0.25) (layer F.Cu) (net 3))
 (via (at 112.2 106.1) (size 1) (drill 0.6) (layers F.Cu B.Cu) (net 3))
 (segment (start 112.2 103.52) (end 112.15 103.47) (width 0.25) (layer B.Cu) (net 3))
 (segment (start 112.2 103.52) (end 112.2 106.1) (width 0.25) (layer B.Cu) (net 3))
 (segment (start 148 112.25) (end 148 113.5) (width 0.6) (layer F.Cu) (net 3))
 (segment (start 145.5 112.5) (end 147 112.5) (width 0.6) (layer F.Cu) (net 3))
 (segment (start 148.24 113.74) (end 148.24 115.38) (width 0.6) (layer F.Cu) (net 3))
 (segment (start 147 112.5) (end 148 113.5) (width 0.6) (layer F.Cu) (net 3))
 (segment (start 148 113.5) (end 148.24 113.74) (width 0.6) (layer F.Cu) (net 3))
 (segment (start 110.91 102.23) (end 112.15 103.47) (width 1) (layer B.Cu) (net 3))
 (segment (start 112.15 103.47) (end 112.15 103.7) (width 1) (layer B.Cu) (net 3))
 (segment (start 109.65 102.23) (end 109.65 103.35) (width 1) (layer F.Cu) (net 3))
 (segment (start 109.65 103.35) (end 109.65 103.25) (width 1) (layer F.Cu) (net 3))
 (segment (start 108.37 102.23) (end 109.65 102.23) (width 1.8) (layer F.Cu) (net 3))
 (segment (start 109.65 102.23) (end 110.91 102.23) (width 1.8) (layer F.Cu) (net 3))
 (segment (start 103.34 112.4) (end 103.34 112.69) (width 1) (layer F.Cu) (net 4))
 (segment (start 103.34 112.69) (end 106.6 115.95) (width 1) (layer F.Cu) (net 4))
 (segment (start 106.6 115.95) (end 119.15 115.95) (width 1) (layer F.Cu) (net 4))
 (segment (start 153.32 123) (end 153.32 122.67) (width 1) (layer B.Cu) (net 4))
 (segment (start 153.32 122.67) (end 151.55 120.9) (width 1) (layer B.Cu) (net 4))
 (segment (start 122.65 115.95) (end 126.2 112.4) (width 1) (layer F.Cu) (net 4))
 (segment (start 119.15 115.95) (end 122.65 115.95) (width 1) (layer F.Cu) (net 4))
 (segment (start 112.2 122.9) (end 119.15 115.95) (width 1) (layer F.Cu) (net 4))
 (via (at 112.2 122.9) (size 1) (drill 0.6) (layers F.Cu B.Cu) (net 4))
 (segment (start 130.15 122.9) (end 112.2 122.9) (width 1) (layer B.Cu) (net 4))
 (segment (start 132.15 120.9) (end 130.15 122.9) (width 1) (layer B.Cu) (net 4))
 (segment (start 151.55 120.9) (end 132.15 120.9) (width 1) (layer B.Cu) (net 4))
 (segment (start 103.34 112.4) (end 103.34 111.61) (width 1.8) (layer B.Cu) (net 4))
 (segment (start 103.34 111.61) (end 108.37 106.58) (width 1.8) (layer B.Cu) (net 4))
 (segment (start 108.37 106.58) (end 108.37 104.77) (width 1.8) (layer B.Cu) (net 4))
 (segment (start 115.7 107.8) (end 111.4 107.8) (width 1) (layer B.Cu) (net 4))
 (segment (start 126.26 107.2) (end 116.3 107.2) (width 0.35) (layer F.Cu) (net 4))
 (segment (start 116.3 107.2) (end 115.7 107.8) (width 0.35) (layer F.Cu) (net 4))
 (via (at 115.7 107.8) (size 1) (drill 0.6) (layers F.Cu B.Cu) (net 4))
 (segment (start 128.69 104.77) (end 126.26 107.2) (width 0.35) (layer F.Cu) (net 4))
 (segment (start 111.4 107.8) (end 108.37 104.77) (width 1) (layer B.Cu) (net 4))
 (segment (start 153.32 123) (end 153.32 122.42) (width 1) (layer B.Cu) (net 4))
 (segment (start 153.32 123) (end 153.32 124.93) (width 0.6) (layer F.Cu) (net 4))
 (segment (start 153.32 124.93) (end 152.75 125.5) (width 0.6) (layer F.Cu) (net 4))
 (segment (start 150.78 115.38) (end 150.78 114.57) (width 1.8) (layer F.Cu) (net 14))
 (segment (start 150.78 114.57) (end 152.39 112.96) (width 1.8) (layer F.Cu) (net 14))
 (segment (start 152.39 112.96) (end 163 112.96) (width 1.8) (layer F.Cu) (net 14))
 (segment (start 145.7 115.38) (end 145.7 115.4) (width 0.6) (layer F.Cu) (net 15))
 (segment (start 128.71 120.05) (end 123.66 125.1) (width 0.6) (layer F.Cu) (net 15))
 (segment (start 141.05 120.05) (end 128.71 120.05) (width 0.6) (layer F.Cu) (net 15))
 (segment (start 145.7 115.4) (end 141.05 120.05) (width 0.6) (layer F.Cu) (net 15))
 (segment (start 143.16 115.38) (end 143.16 115.44) (width 0.6) (layer F.Cu) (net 16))
 (segment (start 124.58 119.1) (end 118.58 125.1) (width 0.6) (layer F.Cu) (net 16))
 (segment (start 139.5 119.1) (end 124.58 119.1) (width 0.6) (layer F.Cu) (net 16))
 (segment (start 143.16 115.44) (end 139.5 119.1) (width 0.6) (layer F.Cu) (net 16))
 (segment (start 140.62 115.38) (end 140.62 115.23) (width 0.6) (layer F.Cu) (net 17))
 (segment (start 122.99 118.15) (end 116.04 125.1) (width 0.6) (layer F.Cu) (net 17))
 (segment (start 137.7 118.15) (end 122.99 118.15) (width 0.6) (layer F.Cu) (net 17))
 (segment (start 140.62 115.23) (end 137.7 118.15) (width 0.6) (layer F.Cu) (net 17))
 (segment (start 113.5 125.1) (end 121.4 117.2) (width 0.6) (layer F.Cu) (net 18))
 (segment (start 133.72 117.2) (end 135.54 115.38) (width 0.6) (layer F.Cu) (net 18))
 (segment (start 121.4 117.2) (end 133.72 117.2) (width 0.6) (layer F.Cu) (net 18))
 (segment (start 125.8 120.4) (end 127.98 120.4) (width 0.6) (layer B.Cu) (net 19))
 (segment (start 125.8 120.42) (end 125.8 120.4) (width 0.6) (layer F.Cu) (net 19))
 (via (at 125.8 120.4) (size 1) (drill 0.6) (layers F.Cu B.Cu) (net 19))
 (segment (start 121.12 125.1) (end 125.8 120.42) (width 0.6) (layer F.Cu) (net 19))
 (segment (start 127.98 120.4) (end 133 115.38) (width 0.6) (layer B.Cu) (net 19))
 (segment (start 110.96 125.1) (end 112.86 127) (width 0.6) (layer F.Cu) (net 12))
 (segment (start 112.86 127) (end 129 127) (width 0.6) (layer F.Cu) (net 12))
 (segment (start 129 127) (end 133 123) (width 0.6) (layer F.Cu) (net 12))
 (segment (start 108.42 125.1) (end 111.47 128.15) (width 1) (layer F.Cu) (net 13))
 (segment (start 143.85 128.15) (end 148.24 123.76) (width 1) (layer F.Cu) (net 13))
 (segment (start 111.47 128.15) (end 143.85 128.15) (width 1) (layer F.Cu) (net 13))
 (segment (start 148.24 123.76) (end 148.24 123) (width 1) (layer F.Cu) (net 13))
 (segment (start 108.42 112.4) (end 115.99 104.83) (width 0.6) (layer F.Cu) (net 5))
 (segment (start 115.99 104.83) (end 115.99 104.77) (width 0.6) (layer F.Cu) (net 5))
 (segment (start 123.66 112.4) (end 125.46 110.6) (width 0.35) (layer F.Cu) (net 11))
 (segment (start 137.6 103.48) (end 138.85 102.23) (width 1) (layer F.Cu) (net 11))
 (segment (start 137.6 103.48) (end 137.6 103.7) (width 1) (layer F.Cu) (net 11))
 (segment (start 137.6 105.8) (end 137.6 103.7) (width 0.25) (layer F.Cu) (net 11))
 (segment (start 132.8 110.6) (end 137.6 105.8) (width 0.35) (layer F.Cu) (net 11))
 (segment (start 125.46 110.6) (end 132.8 110.6) (width 0.35) (layer F.Cu) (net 11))
 (segment (start 118.58 112.4) (end 121.73 109.25) (width 0.35) (layer F.Cu) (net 9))
 (segment (start 135.05 105.85) (end 135.05 103.49) (width 0.25) (layer F.Cu) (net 9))
 (segment (start 131.65 109.25) (end 135.05 105.85) (width 0.35) (layer F.Cu) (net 9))
 (segment (start 121.73 109.25) (end 131.65 109.25) (width 0.35) (layer F.Cu) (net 9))
 (segment (start 135.05 103.49) (end 135.05 103.7) (width 0.25) (layer F.Cu) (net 9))
 (segment (start 136.31 102.23) (end 135.05 103.49) (width 1) (layer F.Cu) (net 9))
 (segment (start 135.05 103.49) (end 135.05 103.7) (width 1) (layer F.Cu) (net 9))
 (segment (start 116.04 112.4) (end 119.89 108.55) (width 0.35) (layer F.Cu) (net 8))
 (segment (start 129.99 108.55) (end 133.77 104.77) (width 0.35) (layer F.Cu) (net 8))
 (segment (start 119.89 108.55) (end 129.99 108.55) (width 0.35) (layer F.Cu) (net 8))
 (segment (start 113.5 112.4) (end 118.05 107.85) (width 0.35) (layer F.Cu) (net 6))
 (segment (start 128.15 107.85) (end 131.23 104.77) (width 0.35) (layer F.Cu) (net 6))
 (segment (start 118.05 107.85) (end 128.15 107.85) (width 0.35) (layer F.Cu) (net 6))
 (segment (start 121.12 112.4) (end 123.62 109.9) (width 0.35) (layer F.Cu) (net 10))
 (segment (start 136.31 105.64) (end 136.31 104.77) (width 0.35) (layer F.Cu) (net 10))
 (segment (start 132.05 109.9) (end 136.31 105.64) (width 0.35) (layer F.Cu) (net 10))
 (segment (start 123.62 109.9) (end 132.05 109.9) (width 0.35) (layer F.Cu) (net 10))
 (segment (start 116.81 106.55) (end 115.45 106.55) (width 0.35) (layer F.Cu) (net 7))
 (segment (start 116.81 106.55) (end 124.25 106.55) (width 0.35) (layer F.Cu) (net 7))
 (segment (start 124.25 106.55) (end 124.9 105.9) (width 0.35) (layer F.Cu) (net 7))
 (segment (start 132.3 103.5) (end 129.5 103.5) (width 0.25) (layer F.Cu) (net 7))
 (segment (start 132.5 103.5) (end 132.3 103.5) (width 1) (layer F.Cu) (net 7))
 (segment (start 133.77 102.23) (end 132.5 103.5) (width 1) (layer F.Cu) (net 7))
 (segment (start 124.9 104.1) (end 124.9 105.9) (width 0.25) (layer F.Cu) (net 7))
 (segment (start 125.5 103.5) (end 124.9 104.1) (width 0.25) (layer F.Cu) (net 7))
 (segment (start 129.5 103.5) (end 125.5 103.5) (width 0.25) (layer F.Cu) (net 7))
 (segment (start 110.96 111.04) (end 110.96 112.4) (width 0.35) (layer F.Cu) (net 7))
 (segment (start 115.45 106.55) (end 110.96 111.04) (width 0.35) (layer F.Cu) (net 7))
 (segment (start 138.08 115.38) (end 138.08 113.02) (width 0.6) (layer F.Cu) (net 1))
 (segment (start 138.08 113.02) (end 138.1 113) (width 0.6) (layer F.Cu) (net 1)))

